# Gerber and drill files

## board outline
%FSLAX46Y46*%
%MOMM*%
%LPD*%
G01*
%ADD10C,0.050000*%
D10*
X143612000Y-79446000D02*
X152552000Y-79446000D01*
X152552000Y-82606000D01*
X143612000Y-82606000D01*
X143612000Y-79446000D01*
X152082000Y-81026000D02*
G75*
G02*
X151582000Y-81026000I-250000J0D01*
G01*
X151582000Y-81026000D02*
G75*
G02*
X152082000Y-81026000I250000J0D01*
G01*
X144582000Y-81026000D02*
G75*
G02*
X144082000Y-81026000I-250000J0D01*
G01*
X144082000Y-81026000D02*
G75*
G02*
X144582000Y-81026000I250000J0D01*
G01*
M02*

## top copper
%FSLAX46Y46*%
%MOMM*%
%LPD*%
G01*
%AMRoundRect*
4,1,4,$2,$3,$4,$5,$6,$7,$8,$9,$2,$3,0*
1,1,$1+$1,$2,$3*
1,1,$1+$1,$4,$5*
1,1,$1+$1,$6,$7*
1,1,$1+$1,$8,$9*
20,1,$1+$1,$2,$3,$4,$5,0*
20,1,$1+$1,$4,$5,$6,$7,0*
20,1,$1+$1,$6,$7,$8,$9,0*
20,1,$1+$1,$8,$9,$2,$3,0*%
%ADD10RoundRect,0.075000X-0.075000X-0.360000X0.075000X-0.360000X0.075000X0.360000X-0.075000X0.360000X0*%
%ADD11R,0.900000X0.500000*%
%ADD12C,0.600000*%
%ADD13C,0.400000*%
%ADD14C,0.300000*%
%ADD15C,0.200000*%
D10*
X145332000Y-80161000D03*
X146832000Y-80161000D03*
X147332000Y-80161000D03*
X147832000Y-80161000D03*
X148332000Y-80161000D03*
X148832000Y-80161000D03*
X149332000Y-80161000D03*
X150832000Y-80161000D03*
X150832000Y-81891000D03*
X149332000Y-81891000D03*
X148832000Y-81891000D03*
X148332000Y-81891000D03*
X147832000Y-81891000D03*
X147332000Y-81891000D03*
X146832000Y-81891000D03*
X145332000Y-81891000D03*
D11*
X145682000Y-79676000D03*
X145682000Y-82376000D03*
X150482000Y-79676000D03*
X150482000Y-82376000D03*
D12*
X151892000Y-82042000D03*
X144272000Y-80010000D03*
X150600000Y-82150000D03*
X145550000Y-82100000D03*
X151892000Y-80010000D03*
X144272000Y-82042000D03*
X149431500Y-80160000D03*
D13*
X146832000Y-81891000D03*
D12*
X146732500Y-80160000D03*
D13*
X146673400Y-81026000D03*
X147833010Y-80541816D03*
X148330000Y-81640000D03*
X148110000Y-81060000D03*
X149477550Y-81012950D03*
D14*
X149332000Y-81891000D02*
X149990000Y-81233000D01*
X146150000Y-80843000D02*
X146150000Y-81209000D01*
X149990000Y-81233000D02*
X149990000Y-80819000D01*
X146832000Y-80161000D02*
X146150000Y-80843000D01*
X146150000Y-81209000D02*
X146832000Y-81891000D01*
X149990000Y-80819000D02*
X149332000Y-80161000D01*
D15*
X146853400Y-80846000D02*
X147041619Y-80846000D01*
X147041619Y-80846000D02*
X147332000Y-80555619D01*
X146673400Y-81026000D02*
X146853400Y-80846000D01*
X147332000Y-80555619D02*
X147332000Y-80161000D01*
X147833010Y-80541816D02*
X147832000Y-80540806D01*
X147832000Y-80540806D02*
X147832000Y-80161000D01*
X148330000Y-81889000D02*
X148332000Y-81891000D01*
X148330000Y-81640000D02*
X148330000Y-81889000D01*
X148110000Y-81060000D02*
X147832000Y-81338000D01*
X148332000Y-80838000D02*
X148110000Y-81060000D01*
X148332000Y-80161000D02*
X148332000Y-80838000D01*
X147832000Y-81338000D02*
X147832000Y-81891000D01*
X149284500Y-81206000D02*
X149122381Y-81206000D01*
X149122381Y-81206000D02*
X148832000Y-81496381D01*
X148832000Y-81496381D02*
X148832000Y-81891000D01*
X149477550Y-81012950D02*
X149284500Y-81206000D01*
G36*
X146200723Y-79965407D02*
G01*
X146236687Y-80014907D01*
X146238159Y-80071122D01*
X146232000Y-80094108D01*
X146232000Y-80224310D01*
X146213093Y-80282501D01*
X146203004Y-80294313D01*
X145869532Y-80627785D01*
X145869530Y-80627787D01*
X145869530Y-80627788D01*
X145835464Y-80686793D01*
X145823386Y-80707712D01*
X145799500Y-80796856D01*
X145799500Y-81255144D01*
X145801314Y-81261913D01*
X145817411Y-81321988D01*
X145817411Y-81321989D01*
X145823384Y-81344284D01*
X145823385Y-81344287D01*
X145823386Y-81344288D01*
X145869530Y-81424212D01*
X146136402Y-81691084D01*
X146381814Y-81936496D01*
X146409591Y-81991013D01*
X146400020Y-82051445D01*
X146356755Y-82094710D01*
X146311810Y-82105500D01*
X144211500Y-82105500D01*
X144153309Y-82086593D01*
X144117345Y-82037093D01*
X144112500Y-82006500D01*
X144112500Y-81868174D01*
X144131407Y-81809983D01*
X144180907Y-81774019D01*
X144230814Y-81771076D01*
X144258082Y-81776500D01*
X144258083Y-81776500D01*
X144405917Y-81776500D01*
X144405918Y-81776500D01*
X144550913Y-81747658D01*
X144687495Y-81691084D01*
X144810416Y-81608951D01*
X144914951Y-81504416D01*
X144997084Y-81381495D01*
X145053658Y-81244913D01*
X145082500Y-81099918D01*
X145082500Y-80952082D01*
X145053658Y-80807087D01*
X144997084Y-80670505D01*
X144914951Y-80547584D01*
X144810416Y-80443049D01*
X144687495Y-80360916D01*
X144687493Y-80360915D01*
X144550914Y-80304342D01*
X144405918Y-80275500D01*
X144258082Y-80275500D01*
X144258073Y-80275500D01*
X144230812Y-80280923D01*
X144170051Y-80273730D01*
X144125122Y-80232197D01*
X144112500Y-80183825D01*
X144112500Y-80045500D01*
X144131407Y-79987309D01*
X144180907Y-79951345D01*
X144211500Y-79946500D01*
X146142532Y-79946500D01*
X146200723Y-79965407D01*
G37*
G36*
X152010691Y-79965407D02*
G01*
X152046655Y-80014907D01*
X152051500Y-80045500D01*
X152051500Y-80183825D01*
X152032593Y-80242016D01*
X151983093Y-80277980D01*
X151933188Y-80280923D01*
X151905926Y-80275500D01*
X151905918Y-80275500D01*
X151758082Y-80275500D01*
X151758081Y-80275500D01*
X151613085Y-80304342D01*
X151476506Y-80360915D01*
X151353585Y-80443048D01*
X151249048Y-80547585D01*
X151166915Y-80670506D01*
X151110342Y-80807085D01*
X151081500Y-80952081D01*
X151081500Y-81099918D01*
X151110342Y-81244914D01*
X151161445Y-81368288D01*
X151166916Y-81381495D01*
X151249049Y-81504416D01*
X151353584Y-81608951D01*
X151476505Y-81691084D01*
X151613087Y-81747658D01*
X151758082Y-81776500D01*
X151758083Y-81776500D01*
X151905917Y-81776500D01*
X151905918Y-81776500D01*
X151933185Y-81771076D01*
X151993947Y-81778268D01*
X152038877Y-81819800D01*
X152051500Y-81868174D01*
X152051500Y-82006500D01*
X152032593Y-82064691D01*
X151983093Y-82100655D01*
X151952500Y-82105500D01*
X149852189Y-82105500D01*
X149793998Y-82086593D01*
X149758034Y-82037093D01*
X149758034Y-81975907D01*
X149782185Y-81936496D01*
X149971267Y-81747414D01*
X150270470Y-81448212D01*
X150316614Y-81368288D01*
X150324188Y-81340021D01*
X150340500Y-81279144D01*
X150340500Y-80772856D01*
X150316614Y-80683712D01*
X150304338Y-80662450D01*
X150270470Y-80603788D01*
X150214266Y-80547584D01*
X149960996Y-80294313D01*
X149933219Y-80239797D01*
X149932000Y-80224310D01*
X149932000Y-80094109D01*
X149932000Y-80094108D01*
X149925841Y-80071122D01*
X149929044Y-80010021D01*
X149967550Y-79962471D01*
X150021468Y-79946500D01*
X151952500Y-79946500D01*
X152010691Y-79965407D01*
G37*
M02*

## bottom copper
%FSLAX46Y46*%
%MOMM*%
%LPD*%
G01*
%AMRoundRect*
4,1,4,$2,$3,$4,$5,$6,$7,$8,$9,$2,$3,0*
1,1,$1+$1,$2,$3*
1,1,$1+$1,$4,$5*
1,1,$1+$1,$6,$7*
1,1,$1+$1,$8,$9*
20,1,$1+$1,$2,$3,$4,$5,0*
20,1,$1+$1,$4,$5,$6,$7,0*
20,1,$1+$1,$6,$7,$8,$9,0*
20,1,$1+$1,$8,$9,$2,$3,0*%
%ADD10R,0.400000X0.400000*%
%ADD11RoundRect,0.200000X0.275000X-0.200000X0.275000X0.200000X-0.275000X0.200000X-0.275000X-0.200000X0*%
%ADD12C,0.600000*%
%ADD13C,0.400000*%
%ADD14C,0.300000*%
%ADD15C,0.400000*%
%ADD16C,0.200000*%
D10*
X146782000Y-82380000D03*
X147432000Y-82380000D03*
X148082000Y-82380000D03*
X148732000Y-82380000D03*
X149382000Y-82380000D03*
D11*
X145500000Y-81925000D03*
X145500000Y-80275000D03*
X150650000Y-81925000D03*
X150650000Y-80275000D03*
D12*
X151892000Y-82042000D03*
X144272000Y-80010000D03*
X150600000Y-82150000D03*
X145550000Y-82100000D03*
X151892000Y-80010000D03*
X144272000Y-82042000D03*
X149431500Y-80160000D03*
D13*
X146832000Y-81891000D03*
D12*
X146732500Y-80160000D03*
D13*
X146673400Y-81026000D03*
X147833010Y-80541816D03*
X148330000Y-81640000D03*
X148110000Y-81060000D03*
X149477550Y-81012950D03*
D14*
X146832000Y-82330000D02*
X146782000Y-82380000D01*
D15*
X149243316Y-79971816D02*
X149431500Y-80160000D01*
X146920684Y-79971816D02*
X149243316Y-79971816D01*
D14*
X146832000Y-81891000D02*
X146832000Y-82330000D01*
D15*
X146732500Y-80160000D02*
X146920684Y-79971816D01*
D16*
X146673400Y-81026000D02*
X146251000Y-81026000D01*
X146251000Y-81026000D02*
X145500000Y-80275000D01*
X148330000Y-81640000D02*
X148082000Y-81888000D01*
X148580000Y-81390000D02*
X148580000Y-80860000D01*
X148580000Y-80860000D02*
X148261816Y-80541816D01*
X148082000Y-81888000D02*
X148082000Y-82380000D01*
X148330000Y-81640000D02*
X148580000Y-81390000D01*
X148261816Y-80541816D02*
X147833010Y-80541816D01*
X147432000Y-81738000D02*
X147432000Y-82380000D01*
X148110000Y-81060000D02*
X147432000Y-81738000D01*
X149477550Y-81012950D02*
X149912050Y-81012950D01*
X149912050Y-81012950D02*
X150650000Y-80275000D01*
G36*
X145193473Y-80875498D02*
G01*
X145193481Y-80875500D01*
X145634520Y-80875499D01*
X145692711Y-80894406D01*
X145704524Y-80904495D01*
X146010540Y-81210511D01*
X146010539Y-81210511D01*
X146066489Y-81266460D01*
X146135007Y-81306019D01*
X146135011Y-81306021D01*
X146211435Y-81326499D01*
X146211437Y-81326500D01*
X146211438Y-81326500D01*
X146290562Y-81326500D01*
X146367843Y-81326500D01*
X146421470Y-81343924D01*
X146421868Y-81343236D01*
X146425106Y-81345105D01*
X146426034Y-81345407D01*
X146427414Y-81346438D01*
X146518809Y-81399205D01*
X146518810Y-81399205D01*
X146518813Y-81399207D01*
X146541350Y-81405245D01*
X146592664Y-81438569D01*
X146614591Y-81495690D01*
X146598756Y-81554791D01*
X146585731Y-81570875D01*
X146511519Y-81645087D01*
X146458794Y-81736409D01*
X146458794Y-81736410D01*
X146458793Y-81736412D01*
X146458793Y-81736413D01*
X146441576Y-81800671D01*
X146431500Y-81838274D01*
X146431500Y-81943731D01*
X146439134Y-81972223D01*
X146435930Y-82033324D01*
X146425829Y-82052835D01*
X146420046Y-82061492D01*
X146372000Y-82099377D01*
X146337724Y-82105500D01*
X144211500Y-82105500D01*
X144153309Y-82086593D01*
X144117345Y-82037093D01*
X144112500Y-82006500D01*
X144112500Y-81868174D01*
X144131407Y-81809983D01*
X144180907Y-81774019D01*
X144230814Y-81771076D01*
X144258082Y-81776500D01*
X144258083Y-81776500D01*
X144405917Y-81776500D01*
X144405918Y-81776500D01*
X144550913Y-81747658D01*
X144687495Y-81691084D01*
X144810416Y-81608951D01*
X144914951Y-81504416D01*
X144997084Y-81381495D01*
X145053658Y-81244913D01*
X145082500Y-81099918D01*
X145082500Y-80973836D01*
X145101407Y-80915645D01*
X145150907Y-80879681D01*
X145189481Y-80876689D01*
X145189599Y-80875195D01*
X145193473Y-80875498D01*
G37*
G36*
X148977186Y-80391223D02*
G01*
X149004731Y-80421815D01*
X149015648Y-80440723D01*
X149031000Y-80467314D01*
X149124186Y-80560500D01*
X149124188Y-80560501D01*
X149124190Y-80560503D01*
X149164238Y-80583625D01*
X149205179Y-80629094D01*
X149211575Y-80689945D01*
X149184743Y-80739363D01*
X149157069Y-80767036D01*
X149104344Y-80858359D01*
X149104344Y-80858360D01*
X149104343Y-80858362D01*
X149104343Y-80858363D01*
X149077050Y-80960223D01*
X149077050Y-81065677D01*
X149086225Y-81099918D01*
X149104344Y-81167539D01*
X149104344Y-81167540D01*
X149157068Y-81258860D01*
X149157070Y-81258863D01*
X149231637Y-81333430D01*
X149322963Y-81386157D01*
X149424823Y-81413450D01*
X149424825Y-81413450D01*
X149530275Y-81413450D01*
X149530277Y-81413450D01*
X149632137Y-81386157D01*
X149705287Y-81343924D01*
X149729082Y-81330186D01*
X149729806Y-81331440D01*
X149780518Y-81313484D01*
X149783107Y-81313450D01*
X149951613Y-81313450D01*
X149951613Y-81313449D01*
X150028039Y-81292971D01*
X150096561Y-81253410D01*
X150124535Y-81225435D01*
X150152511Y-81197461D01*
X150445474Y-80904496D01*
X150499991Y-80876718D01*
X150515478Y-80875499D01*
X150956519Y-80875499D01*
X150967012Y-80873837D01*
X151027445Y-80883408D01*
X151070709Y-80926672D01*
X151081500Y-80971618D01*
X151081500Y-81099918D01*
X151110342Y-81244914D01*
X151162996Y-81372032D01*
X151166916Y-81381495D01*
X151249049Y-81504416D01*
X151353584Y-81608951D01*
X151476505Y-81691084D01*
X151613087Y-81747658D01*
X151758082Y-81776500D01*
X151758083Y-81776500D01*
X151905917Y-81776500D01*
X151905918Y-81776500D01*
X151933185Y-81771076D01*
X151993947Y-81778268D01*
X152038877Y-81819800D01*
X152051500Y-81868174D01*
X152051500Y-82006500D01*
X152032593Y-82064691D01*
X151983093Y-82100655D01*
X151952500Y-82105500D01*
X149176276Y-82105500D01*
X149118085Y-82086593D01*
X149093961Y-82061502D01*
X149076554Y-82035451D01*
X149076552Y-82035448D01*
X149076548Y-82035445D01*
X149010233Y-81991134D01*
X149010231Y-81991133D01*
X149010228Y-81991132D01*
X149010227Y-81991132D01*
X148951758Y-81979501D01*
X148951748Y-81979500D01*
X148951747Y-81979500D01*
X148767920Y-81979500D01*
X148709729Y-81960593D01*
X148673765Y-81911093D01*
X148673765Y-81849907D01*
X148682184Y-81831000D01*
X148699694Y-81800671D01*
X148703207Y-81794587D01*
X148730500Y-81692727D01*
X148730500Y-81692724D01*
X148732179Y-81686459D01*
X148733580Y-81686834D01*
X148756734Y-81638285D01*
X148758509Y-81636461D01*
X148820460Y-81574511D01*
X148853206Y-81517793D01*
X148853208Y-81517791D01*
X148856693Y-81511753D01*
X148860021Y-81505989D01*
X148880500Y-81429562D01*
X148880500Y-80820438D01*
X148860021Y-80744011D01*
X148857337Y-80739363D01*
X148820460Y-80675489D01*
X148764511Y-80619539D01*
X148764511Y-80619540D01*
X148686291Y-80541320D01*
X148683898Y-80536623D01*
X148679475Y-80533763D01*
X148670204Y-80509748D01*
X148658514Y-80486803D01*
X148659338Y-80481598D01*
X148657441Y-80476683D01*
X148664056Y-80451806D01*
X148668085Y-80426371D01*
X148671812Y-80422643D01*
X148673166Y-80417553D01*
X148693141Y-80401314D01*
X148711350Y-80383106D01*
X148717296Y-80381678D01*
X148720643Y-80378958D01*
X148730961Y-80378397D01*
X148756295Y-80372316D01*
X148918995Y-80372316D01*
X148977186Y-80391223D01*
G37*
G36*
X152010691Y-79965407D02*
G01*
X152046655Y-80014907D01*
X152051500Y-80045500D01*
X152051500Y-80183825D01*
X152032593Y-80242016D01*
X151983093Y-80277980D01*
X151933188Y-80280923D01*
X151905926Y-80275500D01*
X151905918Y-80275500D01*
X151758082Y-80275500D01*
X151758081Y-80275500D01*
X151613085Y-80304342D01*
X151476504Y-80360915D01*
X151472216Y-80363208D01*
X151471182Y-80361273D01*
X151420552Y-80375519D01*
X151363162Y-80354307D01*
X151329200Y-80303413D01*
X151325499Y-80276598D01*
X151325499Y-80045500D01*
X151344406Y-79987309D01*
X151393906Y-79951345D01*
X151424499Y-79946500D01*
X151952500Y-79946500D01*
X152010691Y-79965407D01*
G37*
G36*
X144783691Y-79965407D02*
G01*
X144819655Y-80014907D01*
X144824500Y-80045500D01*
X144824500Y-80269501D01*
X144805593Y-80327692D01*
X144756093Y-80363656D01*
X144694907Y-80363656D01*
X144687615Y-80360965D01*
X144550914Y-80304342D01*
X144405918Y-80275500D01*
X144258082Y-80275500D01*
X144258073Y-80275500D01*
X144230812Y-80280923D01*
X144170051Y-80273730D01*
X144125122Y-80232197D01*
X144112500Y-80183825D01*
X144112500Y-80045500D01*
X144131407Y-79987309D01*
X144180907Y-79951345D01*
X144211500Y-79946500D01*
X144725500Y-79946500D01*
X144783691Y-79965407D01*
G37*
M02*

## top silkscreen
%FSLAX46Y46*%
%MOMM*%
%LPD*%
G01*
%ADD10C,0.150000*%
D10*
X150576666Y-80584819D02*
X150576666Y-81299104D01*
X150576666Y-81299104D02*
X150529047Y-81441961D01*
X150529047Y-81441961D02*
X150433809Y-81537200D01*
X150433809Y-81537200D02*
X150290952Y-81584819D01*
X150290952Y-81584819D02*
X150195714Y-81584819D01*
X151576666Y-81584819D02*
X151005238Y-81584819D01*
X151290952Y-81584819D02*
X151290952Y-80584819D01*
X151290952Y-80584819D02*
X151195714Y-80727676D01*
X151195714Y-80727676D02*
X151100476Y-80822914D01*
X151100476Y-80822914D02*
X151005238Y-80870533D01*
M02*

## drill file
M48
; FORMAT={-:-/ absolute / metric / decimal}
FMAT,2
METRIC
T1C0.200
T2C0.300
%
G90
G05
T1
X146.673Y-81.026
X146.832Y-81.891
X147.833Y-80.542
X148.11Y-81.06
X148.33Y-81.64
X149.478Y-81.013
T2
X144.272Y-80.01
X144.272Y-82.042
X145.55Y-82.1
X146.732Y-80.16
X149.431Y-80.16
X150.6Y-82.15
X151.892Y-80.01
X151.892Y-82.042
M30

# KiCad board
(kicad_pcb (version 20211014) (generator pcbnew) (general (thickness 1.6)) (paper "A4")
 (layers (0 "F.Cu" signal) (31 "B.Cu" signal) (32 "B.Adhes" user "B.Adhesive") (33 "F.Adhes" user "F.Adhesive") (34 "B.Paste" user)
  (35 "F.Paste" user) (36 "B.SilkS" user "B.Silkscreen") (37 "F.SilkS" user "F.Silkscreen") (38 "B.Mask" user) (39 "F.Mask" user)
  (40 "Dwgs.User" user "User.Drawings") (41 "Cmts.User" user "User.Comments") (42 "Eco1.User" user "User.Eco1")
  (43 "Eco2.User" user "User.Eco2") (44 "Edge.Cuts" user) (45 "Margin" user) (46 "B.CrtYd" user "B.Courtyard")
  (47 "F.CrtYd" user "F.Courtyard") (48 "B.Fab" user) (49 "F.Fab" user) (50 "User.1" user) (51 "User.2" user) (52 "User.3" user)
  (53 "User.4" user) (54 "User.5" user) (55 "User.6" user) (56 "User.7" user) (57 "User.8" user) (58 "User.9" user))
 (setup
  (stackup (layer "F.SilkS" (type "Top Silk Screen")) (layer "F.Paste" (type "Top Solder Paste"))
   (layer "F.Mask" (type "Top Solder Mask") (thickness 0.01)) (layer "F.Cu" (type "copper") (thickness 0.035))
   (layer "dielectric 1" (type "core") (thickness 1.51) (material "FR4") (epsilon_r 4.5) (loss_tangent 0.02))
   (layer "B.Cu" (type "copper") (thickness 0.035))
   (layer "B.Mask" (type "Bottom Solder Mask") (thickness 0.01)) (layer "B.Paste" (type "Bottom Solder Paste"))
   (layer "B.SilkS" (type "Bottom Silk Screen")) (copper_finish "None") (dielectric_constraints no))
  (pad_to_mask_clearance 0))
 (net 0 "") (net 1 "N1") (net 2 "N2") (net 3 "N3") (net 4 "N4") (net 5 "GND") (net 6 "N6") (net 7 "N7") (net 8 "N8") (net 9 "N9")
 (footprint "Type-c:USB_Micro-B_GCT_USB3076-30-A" (layer "F.Cu") (at 148.082 82.38 180)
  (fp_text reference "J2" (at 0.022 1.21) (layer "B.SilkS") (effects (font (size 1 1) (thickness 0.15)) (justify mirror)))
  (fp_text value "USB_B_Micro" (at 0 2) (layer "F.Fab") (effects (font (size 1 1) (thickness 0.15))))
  (pad "1" smd rect (at 1.3 0 180) (size 0.4 0.4) (layers "B.Cu" "B.Paste" "B.Mask") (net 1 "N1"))
  (pad "2" smd rect (at 0.65 0 180) (size 0.4 0.4) (layers "B.Cu" "B.Paste" "B.Mask") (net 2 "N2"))
  (pad "3" smd rect (at 0 0 180) (size 0.4 0.4) (layers "B.Cu" "B.Paste" "B.Mask") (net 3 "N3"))
  (pad "4" smd rect (at -0.65 0 180) (size 0.4 0.4) (layers "B.Cu" "B.Paste" "B.Mask") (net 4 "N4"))
  (pad "5" smd rect (at -1.3 0 180) (size 0.4 0.4) (layers "B.Cu" "B.Paste" "B.Mask") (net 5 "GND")))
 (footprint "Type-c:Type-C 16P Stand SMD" (layer "F.Cu") (at 148.082 81.026)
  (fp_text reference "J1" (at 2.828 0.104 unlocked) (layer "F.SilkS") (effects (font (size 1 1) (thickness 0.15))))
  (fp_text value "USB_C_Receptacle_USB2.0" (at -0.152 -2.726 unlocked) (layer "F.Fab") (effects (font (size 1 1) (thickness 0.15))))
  (fp_rect (start -4.47 -1.58) (end 4.47 1.58) (layer "Edge.Cuts") (width 0.05) (fill none))
  (fp_circle (center 3.75 0) (end 4 0) (layer "Edge.Cuts") (width 0.05) (fill none))
  (fp_circle (center -3.75 0) (end -3.5 0) (layer "Edge.Cuts") (width 0.05) (fill none))
  (pad "A1" smd roundrect (at -2.75 -0.865) (size 0.3 0.87) (layers "F.Cu" "F.Paste" "F.Mask") (roundrect_rratio 0.25) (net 5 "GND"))
  (pad "A4" smd roundrect (at -1.25 -0.865) (size 0.3 0.87) (layers "F.Cu" "F.Paste" "F.Mask") (roundrect_rratio 0.25) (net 1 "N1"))
  (pad "A5" smd roundrect (at -0.75 -0.865) (size 0.3 0.87) (layers "F.Cu" "F.Paste" "F.Mask") (roundrect_rratio 0.25) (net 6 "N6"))
  (pad "A6" smd roundrect (at -0.25 -0.865) (size 0.3 0.87) (layers "F.Cu" "F.Paste" "F.Mask") (roundrect_rratio 0.25) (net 3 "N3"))
  (pad "A7" smd roundrect (at 0.25 -0.865) (size 0.3 0.87) (layers "F.Cu" "F.Paste" "F.Mask") (roundrect_rratio 0.25) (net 2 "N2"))
  (pad "A8" smd roundrect (at 0.75 -0.865) (size 0.3 0.87) (layers "F.Cu" "F.Paste" "F.Mask") (roundrect_rratio 0.25) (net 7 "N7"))
  (pad "A9" smd roundrect (at 1.25 -0.865) (size 0.3 0.87) (layers "F.Cu" "F.Paste" "F.Mask") (roundrect_rratio 0.25) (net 1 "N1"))
  (pad "A12" smd roundrect (at 2.75 -0.865) (size 0.3 0.87) (layers "F.Cu" "F.Paste" "F.Mask") (roundrect_rratio 0.25) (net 5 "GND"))
  (pad "B1" smd roundrect (at 2.75 0.865) (size 0.3 0.87) (layers "F.Cu" "F.Paste" "F.Mask") (roundrect_rratio 0.25) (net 5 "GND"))
  (pad "B4" smd roundrect (at 1.25 0.865) (size 0.3 0.87) (layers "F.Cu" "F.Paste" "F.Mask") (roundrect_rratio 0.25) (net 1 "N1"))
  (pad "B5" smd roundrect (at 0.75 0.865) (size 0.3 0.87) (layers "F.Cu" "F.Paste" "F.Mask") (roundrect_rratio 0.25) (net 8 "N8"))
  (pad "B6" smd roundrect (at 0.25 0.865) (size 0.3 0.87) (layers "F.Cu" "F.Paste" "F.Mask") (roundrect_rratio 0.25) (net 3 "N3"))
  (pad "B7" smd roundrect (at -0.25 0.865) (size 0.3 0.87) (layers "F.Cu" "F.Paste" "F.Mask") (roundrect_rratio 0.25) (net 2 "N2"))
  (pad "B8" smd roundrect (at -0.75 0.865) (size 0.3 0.87) (layers "F.Cu" "F.Paste" "F.Mask") (roundrect_rratio 0.25) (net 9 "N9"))
  (pad "B9" smd roundrect (at -1.25 0.865) (size 0.3 0.87) (layers "F.Cu" "F.Paste" "F.Mask") (roundrect_rratio 0.25) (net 1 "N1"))
  (pad "B12" smd roundrect (at -2.75 0.865) (size 0.3 0.87) (layers "F.Cu" "F.Paste" "F.Mask") (roundrect_rratio 0.25) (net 5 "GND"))
  (pad "S1" smd rect (at -2.4 -1.35) (size 0.9 0.5) (layers "F.Cu" "F.Paste" "F.Mask") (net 5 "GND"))
  (pad "S1" smd rect (at -2.4 1.35) (size 0.9 0.5) (layers "F.Cu" "F.Paste" "F.Mask") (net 5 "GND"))
  (pad "S1" smd rect (at 2.4 -1.35) (size 0.9 0.5) (layers "F.Cu" "F.Paste" "F.Mask") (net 5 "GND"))
  (pad "S1" smd rect (at 2.4 1.35) (size 0.9 0.5) (layers "F.Cu" "F.Paste" "F.Mask") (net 5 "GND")))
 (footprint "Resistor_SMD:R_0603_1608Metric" (layer "B.Cu") (at 145.5 81.1 90)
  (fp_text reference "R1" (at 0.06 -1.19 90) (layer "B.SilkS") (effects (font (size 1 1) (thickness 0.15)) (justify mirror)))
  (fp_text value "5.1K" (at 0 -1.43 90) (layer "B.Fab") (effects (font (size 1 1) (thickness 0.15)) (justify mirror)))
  (pad "1" smd roundrect (at -0.825 0 90) (size 0.8 0.95) (layers "B.Cu" "B.Paste" "B.Mask") (roundrect_rratio 0.25) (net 5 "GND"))
  (pad "2" smd roundrect (at 0.825 0 90) (size 0.8 0.95) (layers "B.Cu" "B.Paste" "B.Mask") (roundrect_rratio 0.25) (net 6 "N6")))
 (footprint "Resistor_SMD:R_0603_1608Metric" (layer "B.Cu") (at 150.65 81.1 90)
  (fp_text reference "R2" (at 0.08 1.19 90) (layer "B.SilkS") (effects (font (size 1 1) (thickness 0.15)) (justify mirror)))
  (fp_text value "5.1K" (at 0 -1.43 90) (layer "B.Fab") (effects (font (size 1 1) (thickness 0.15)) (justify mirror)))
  (pad "1" smd roundrect (at -0.825 0 90) (size 0.8 0.95) (layers "B.Cu" "B.Paste" "B.Mask") (roundrect_rratio 0.25) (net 5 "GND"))
  (pad "2" smd roundrect (at 0.825 0 90) (size 0.8 0.95) (layers "B.Cu" "B.Paste" "B.Mask") (roundrect_rratio 0.25) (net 8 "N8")))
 (via (at 151.892 82.042) (size 0.6) (drill 0.3) (layers "F.Cu" "B.Cu") (free) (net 5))
 (via (at 144.272 80.01) (size 0.6) (drill 0.3) (layers "F.Cu" "B.Cu") (free) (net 5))
 (via (at 150.6 82.15) (size 0.6) (drill 0.3) (layers "F.Cu" "B.Cu") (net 5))
 (via (at 145.55 82.1) (size 0.6) (drill 0.3) (layers "F.Cu" "B.Cu") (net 5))
 (via (at 151.892 80.01) (size 0.6) (drill 0.3) (layers "F.Cu" "B.Cu") (free) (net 5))
 (via (at 144.272 82.042) (size 0.6) (drill 0.3) (layers "F.Cu" "B.Cu") (free) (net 5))
 (segment (start 149.332 81.891) (end 149.99 81.233) (width 0.3) (layer "F.Cu") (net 1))
 (segment (start 146.15 80.843) (end 146.15 81.209) (width 0.3) (layer "F.Cu") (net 1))
 (segment (start 149.99 81.233) (end 149.99 80.819) (width 0.3) (layer "F.Cu") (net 1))
 (segment (start 146.832 80.161) (end 146.15 80.843) (width 0.3) (layer "F.Cu") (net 1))
 (segment (start 146.15 81.209) (end 146.832 81.891) (width 0.3) (layer "F.Cu") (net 1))
 (segment (start 149.99 80.819) (end 149.332 80.161) (width 0.3) (layer "F.Cu") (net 1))
 (via (at 149.4315 80.16) (size 0.6) (drill 0.3) (layers "F.Cu" "B.Cu") (free) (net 1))
 (via (at 146.832 81.891) (size 0.4) (drill 0.2) (layers "F.Cu" "B.Cu") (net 1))
 (via (at 146.7325 80.16) (size 0.6) (drill 0.3) (layers "F.Cu" "B.Cu") (free) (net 1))
 (segment (start 146.832 82.33) (end 146.782 82.38) (width 0.3) (layer "B.Cu") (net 1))
 (segment (start 149.243316 79.971816) (end 149.4315 80.16) (width 0.4) (layer "B.Cu") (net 1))
 (segment (start 146.920684 79.971816) (end 149.243316 79.971816) (width 0.4) (layer "B.Cu") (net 1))
 (segment (start 146.832 81.891) (end 146.832 82.33) (width 0.3) (layer "B.Cu") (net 1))
 (segment (start 146.7325 80.16) (end 146.920684 79.971816) (width 0.4) (layer "B.Cu") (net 1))
 (segment (start 146.8534 80.846) (end 147.041619 80.846) (width 0.2) (layer "F.Cu") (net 6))
 (segment (start 147.041619 80.846) (end 147.332 80.555619) (width 0.2) (layer "F.Cu") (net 6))
 (segment (start 146.6734 81.026) (end 146.8534 80.846) (width 0.2) (layer "F.Cu") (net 6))
 (segment (start 147.332 80.555619) (end 147.332 80.161) (width 0.2) (layer "F.Cu") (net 6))
 (via (at 146.6734 81.026) (size 0.4) (drill 0.2) (layers "F.Cu" "B.Cu") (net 6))
 (segment (start 146.6734 81.026) (end 146.251 81.026) (width 0.2) (layer "B.Cu") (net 6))
 (segment (start 146.251 81.026) (end 145.5 80.275) (width 0.2) (layer "B.Cu") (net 6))
 (segment (start 147.83301 80.541816) (end 147.832 80.540806) (width 0.2) (layer "F.Cu") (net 3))
 (segment (start 147.832 80.540806) (end 147.832 80.161) (width 0.2) (layer "F.Cu") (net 3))
 (segment (start 148.33 81.889) (end 148.332 81.891) (width 0.2) (layer "F.Cu") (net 3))
 (segment (start 148.33 81.64) (end 148.33 81.889) (width 0.2) (layer "F.Cu") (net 3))
 (via (at 147.83301 80.541816) (size 0.4) (drill 0.2) (layers "F.Cu" "B.Cu") (free) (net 3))
 (via (at 148.33 81.64) (size 0.4) (drill 0.2) (layers "F.Cu" "B.Cu") (free) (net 3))
 (segment (start 148.33 81.64) (end 148.082 81.888) (width 0.2) (layer "B.Cu") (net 3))
 (segment (start 148.58 81.39) (end 148.58 80.86) (width 0.2) (layer "B.Cu") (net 3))
 (segment (start 148.58 80.86) (end 148.261816 80.541816) (width 0.2) (layer "B.Cu") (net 3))
 (segment (start 148.082 81.888) (end 148.082 82.38) (width 0.2) (layer "B.Cu") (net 3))
 (segment (start 148.33 81.64) (end 148.58 81.39) (width 0.2) (layer "B.Cu") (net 3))
 (segment (start 148.261816 80.541816) (end 147.83301 80.541816) (width 0.2) (layer "B.Cu") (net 3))
 (segment (start 148.11 81.06) (end 147.832 81.338) (width 0.2) (layer "F.Cu") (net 2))
 (segment (start 148.332 80.838) (end 148.11 81.06) (width 0.2) (layer "F.Cu") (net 2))
 (segment (start 148.332 80.161) (end 148.332 80.838) (width 0.2) (layer "F.Cu") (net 2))
 (segment (start 147.832 81.338) (end 147.832 81.891) (width 0.2) (layer "F.Cu") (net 2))
 (via (at 148.11 81.06) (size 0.4) (drill 0.2) (layers "F.Cu" "B.Cu") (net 2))
 (segment (start 147.432 81.738) (end 147.432 82.38) (width 0.2) (layer "B.Cu") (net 2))
 (segment (start 148.11 81.06) (end 147.432 81.738) (width 0.2) (layer "B.Cu") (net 2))
 (segment (start 149.2845 81.206) (end 149.122381 81.206) (width 0.2) (layer "F.Cu") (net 8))
 (segment (start 149.122381 81.206) (end 148.832 81.496381) (width 0.2) (layer "F.Cu") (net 8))
 (segment (start 148.832 81.496381) (end 148.832 81.891) (width 0.2) (layer "F.Cu") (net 8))
 (segment (start 149.47755 81.01295) (end 149.2845 81.206) (width 0.2) (layer "F.Cu") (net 8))
 (via (at 149.47755 81.01295) (size 0.4) (drill 0.2) (layers "F.Cu" "B.Cu") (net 8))
 (segment (start 149.47755 81.01295) (end 149.91205 81.01295) (width 0.2) (layer "B.Cu") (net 8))
 (segment (start 149.91205 81.01295) (end 150.65 80.275) (width 0.2) (layer "B.Cu") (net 8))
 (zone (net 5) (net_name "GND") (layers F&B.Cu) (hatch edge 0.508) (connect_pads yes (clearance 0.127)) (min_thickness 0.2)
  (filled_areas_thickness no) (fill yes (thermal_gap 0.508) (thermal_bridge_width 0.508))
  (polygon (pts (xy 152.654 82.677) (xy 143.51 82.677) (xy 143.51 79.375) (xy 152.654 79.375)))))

